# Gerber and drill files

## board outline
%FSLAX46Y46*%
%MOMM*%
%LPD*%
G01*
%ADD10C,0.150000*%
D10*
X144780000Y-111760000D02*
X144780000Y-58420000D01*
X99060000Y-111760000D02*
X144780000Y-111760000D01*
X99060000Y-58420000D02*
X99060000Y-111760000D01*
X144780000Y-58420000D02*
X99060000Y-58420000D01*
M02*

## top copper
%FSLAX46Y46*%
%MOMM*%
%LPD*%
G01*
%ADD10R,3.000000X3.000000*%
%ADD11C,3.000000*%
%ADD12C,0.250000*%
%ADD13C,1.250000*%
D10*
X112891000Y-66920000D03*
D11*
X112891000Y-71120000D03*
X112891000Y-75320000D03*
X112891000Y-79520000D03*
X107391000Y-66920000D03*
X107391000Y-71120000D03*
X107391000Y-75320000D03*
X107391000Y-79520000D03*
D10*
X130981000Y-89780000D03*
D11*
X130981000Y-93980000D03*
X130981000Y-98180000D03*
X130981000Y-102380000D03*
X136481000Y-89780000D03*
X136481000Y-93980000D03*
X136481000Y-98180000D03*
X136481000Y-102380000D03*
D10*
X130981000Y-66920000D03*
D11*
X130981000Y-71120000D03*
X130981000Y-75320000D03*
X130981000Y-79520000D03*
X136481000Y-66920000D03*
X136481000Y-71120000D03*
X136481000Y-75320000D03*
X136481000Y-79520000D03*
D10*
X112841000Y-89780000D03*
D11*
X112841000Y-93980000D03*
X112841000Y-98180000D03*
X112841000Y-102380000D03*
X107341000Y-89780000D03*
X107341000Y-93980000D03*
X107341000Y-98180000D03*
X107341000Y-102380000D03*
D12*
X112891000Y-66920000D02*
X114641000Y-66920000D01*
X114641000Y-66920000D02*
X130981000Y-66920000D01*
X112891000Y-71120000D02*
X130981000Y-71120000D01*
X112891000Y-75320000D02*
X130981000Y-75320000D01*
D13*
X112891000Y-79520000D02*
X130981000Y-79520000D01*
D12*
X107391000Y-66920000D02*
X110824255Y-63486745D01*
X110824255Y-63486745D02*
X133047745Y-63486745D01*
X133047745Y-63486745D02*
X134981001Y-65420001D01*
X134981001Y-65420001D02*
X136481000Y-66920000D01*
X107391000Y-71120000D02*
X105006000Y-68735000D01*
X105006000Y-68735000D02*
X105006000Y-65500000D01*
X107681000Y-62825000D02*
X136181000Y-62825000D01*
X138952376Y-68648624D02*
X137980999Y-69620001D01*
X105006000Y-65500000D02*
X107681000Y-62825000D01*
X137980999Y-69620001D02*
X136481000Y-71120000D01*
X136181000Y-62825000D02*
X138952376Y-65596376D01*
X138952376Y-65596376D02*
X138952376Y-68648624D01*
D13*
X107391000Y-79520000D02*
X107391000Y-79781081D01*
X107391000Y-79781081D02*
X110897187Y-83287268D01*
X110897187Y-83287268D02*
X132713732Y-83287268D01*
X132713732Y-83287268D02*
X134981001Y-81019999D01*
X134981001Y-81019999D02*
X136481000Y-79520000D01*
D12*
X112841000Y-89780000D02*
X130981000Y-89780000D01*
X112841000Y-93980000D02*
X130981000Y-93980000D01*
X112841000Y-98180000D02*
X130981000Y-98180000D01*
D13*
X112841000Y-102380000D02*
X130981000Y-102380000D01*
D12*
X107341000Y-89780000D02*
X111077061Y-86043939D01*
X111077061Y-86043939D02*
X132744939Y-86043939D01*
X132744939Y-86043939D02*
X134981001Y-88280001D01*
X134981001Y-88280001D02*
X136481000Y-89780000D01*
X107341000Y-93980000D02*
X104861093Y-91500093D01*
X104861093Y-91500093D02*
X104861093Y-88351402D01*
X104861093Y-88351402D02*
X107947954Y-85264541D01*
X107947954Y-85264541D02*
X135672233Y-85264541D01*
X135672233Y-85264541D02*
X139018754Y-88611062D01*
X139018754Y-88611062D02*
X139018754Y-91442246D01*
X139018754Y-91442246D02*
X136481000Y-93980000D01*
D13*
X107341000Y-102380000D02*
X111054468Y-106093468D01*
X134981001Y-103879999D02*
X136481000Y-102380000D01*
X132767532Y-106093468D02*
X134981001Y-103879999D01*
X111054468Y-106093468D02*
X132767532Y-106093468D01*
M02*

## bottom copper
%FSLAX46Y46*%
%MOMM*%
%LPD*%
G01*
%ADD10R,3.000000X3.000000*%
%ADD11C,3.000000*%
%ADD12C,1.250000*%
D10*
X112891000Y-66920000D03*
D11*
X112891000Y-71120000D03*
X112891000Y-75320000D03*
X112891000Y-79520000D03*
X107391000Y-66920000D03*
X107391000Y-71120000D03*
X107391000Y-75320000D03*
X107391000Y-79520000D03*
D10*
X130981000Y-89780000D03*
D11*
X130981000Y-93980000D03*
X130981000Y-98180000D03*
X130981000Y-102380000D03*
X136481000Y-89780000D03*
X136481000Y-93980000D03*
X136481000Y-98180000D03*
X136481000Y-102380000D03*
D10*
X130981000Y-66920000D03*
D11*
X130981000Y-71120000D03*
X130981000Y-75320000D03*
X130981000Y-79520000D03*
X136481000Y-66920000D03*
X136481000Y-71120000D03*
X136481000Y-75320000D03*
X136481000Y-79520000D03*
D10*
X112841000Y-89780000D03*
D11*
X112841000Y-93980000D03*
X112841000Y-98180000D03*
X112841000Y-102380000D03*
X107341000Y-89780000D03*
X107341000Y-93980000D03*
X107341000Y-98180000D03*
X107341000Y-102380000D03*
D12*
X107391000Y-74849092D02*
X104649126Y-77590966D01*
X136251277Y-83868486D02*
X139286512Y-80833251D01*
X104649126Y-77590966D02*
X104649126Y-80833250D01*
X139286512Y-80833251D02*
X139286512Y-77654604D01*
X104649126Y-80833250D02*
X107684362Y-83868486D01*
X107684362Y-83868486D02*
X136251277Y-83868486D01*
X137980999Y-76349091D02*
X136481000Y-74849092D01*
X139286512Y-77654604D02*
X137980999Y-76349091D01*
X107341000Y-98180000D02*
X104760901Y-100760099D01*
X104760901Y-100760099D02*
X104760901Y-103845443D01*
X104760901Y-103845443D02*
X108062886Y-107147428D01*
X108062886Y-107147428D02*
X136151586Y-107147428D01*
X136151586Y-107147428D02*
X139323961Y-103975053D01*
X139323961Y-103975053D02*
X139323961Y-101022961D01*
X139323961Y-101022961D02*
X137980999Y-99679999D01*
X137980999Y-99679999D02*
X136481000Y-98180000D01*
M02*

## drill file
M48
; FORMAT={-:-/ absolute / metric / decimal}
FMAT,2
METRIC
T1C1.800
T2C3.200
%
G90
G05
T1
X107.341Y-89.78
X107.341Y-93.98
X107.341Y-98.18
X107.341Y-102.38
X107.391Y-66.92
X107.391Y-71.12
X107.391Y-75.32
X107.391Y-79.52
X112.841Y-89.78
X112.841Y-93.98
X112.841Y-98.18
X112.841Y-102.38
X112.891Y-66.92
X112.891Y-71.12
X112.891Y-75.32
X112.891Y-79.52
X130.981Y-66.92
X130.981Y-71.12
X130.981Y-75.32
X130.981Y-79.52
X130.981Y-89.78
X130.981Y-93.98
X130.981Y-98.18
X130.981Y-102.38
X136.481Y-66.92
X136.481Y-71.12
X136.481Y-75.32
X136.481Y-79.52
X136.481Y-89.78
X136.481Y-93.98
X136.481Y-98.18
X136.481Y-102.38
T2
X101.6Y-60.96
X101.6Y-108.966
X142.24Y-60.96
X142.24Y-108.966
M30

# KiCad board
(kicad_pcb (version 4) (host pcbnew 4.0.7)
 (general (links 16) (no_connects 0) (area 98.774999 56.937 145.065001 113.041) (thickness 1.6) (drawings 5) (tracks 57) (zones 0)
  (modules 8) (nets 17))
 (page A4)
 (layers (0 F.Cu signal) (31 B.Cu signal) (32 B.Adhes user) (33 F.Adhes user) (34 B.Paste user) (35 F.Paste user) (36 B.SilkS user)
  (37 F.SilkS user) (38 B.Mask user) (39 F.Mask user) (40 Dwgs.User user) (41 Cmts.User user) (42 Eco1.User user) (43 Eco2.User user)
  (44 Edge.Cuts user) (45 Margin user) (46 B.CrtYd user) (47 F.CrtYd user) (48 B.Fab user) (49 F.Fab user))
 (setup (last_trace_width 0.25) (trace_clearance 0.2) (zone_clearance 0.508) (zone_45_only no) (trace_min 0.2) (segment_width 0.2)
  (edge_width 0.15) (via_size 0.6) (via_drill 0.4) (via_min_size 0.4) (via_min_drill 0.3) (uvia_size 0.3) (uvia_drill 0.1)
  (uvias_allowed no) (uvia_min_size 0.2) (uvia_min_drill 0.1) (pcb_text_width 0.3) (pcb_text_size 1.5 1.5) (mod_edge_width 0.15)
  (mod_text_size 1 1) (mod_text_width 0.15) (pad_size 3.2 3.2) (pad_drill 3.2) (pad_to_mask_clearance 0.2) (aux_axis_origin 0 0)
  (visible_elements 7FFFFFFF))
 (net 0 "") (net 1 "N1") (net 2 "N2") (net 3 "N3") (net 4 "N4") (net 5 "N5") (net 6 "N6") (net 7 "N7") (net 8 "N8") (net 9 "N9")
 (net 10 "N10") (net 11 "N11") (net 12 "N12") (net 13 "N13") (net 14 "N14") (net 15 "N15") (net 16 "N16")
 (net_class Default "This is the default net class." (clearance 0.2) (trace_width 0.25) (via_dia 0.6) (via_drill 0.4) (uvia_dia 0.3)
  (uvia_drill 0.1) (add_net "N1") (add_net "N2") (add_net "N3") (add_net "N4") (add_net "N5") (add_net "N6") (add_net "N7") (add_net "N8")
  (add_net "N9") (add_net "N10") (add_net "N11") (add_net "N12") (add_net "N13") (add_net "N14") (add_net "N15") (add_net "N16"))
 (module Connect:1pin (layer F.Cu) (at 142.24 108.966)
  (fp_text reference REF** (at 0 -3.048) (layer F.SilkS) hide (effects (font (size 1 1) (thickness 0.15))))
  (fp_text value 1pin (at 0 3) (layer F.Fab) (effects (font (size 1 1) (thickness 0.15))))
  (pad "" np_thru_hole circle (at 0 0) (size 3.2 3.2) (drill 3.2) (layers *.Cu *.Mask)))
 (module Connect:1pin (layer F.Cu) (at 101.6 108.966)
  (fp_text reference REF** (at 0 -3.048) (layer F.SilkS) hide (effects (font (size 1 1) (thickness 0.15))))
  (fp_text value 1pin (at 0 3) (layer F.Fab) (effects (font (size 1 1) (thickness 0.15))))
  (pad "" np_thru_hole circle (at 0 0) (size 3.2 3.2) (drill 3.2) (layers *.Cu *.Mask)))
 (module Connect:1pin (layer F.Cu) (at 101.6 60.96)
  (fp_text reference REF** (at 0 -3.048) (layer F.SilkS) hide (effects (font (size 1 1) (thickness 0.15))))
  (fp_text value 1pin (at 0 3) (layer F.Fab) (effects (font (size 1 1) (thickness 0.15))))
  (pad "" np_thru_hole circle (at 0 0) (size 3.2 3.2) (drill 3.2) (layers *.Cu *.Mask)))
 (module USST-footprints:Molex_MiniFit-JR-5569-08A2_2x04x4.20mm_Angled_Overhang (layer F.Cu) (at 112.891 66.92 270)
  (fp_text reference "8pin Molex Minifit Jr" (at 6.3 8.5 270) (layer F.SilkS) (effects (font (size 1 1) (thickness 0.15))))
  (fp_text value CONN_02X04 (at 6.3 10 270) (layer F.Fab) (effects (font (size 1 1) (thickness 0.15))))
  (pad 1 thru_hole rect (at 0 0 270) (size 3 3) (drill 1.8) (layers *.Cu *.Mask) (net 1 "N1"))
  (pad 2 thru_hole circle (at 4.2 0 270) (size 3 3) (drill 1.8) (layers *.Cu *.Mask) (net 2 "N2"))
  (pad 3 thru_hole circle (at 8.4 0 270) (size 3 3) (drill 1.8) (layers *.Cu *.Mask) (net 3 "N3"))
  (pad 4 thru_hole circle (at 12.6 0 270) (size 3 3) (drill 1.8) (layers *.Cu *.Mask) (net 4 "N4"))
  (pad 5 thru_hole circle (at 0 5.5 270) (size 3 3) (drill 1.8) (layers *.Cu *.Mask) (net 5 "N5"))
  (pad 6 thru_hole circle (at 4.2 5.5 270) (size 3 3) (drill 1.8) (layers *.Cu *.Mask) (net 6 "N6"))
  (pad 7 thru_hole circle (at 8.4 5.5 270) (size 3 3) (drill 1.8) (layers *.Cu *.Mask) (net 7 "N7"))
  (pad 8 thru_hole circle (at 12.6 5.5 270) (size 3 3) (drill 1.8) (layers *.Cu *.Mask) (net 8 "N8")))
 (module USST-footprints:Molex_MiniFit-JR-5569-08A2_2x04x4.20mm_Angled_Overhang (layer B.Cu) (at 130.981 89.78 270)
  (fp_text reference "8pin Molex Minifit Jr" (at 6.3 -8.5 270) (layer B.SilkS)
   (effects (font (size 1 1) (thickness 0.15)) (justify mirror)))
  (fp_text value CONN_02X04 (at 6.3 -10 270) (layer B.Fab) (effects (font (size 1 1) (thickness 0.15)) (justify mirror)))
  (pad 1 thru_hole rect (at 0 0 270) (size 3 3) (drill 1.8) (layers *.Cu *.Mask) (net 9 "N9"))
  (pad 2 thru_hole circle (at 4.2 0 270) (size 3 3) (drill 1.8) (layers *.Cu *.Mask) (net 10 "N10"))
  (pad 3 thru_hole circle (at 8.4 0 270) (size 3 3) (drill 1.8) (layers *.Cu *.Mask) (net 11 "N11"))
  (pad 4 thru_hole circle (at 12.6 0 270) (size 3 3) (drill 1.8) (layers *.Cu *.Mask) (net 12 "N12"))
  (pad 5 thru_hole circle (at 0 -5.5 270) (size 3 3) (drill 1.8) (layers *.Cu *.Mask) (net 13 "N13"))
  (pad 6 thru_hole circle (at 4.2 -5.5 270) (size 3 3) (drill 1.8) (layers *.Cu *.Mask) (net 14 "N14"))
  (pad 7 thru_hole circle (at 8.4 -5.5 270) (size 3 3) (drill 1.8) (layers *.Cu *.Mask) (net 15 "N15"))
  (pad 8 thru_hole circle (at 12.6 -5.5 270) (size 3 3) (drill 1.8) (layers *.Cu *.Mask) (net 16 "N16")))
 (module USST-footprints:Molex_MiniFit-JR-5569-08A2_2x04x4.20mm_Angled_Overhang (layer B.Cu) (at 130.981 66.92 270)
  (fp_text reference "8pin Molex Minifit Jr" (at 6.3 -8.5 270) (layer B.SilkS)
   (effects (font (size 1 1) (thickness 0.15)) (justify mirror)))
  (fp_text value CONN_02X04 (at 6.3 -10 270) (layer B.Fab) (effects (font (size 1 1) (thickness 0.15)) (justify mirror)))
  (pad 1 thru_hole rect (at 0 0 270) (size 3 3) (drill 1.8) (layers *.Cu *.Mask) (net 1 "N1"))
  (pad 2 thru_hole circle (at 4.2 0 270) (size 3 3) (drill 1.8) (layers *.Cu *.Mask) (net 2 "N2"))
  (pad 3 thru_hole circle (at 8.4 0 270) (size 3 3) (drill 1.8) (layers *.Cu *.Mask) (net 3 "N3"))
  (pad 4 thru_hole circle (at 12.6 0 270) (size 3 3) (drill 1.8) (layers *.Cu *.Mask) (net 4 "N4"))
  (pad 5 thru_hole circle (at 0 -5.5 270) (size 3 3) (drill 1.8) (layers *.Cu *.Mask) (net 5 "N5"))
  (pad 6 thru_hole circle (at 4.2 -5.5 270) (size 3 3) (drill 1.8) (layers *.Cu *.Mask) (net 6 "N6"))
  (pad 7 thru_hole circle (at 8.4 -5.5 270) (size 3 3) (drill 1.8) (layers *.Cu *.Mask) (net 7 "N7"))
  (pad 8 thru_hole circle (at 12.6 -5.5 270) (size 3 3) (drill 1.8) (layers *.Cu *.Mask) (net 8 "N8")))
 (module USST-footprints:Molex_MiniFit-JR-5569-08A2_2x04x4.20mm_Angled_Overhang (layer F.Cu) (at 112.841 89.78 270)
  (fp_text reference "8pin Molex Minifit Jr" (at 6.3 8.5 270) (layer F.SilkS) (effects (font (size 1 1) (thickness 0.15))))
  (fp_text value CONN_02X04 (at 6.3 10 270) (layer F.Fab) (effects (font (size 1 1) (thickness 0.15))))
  (pad 1 thru_hole rect (at 0 0 270) (size 3 3) (drill 1.8) (layers *.Cu *.Mask) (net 9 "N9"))
  (pad 2 thru_hole circle (at 4.2 0 270) (size 3 3) (drill 1.8) (layers *.Cu *.Mask) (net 10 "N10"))
  (pad 3 thru_hole circle (at 8.4 0 270) (size 3 3) (drill 1.8) (layers *.Cu *.Mask) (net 11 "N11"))
  (pad 4 thru_hole circle (at 12.6 0 270) (size 3 3) (drill 1.8) (layers *.Cu *.Mask) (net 12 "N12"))
  (pad 5 thru_hole circle (at 0 5.5 270) (size 3 3) (drill 1.8) (layers *.Cu *.Mask) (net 13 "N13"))
  (pad 6 thru_hole circle (at 4.2 5.5 270) (size 3 3) (drill 1.8) (layers *.Cu *.Mask) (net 14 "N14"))
  (pad 7 thru_hole circle (at 8.4 5.5 270) (size 3 3) (drill 1.8) (layers *.Cu *.Mask) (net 15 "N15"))
  (pad 8 thru_hole circle (at 12.6 5.5 270) (size 3 3) (drill 1.8) (layers *.Cu *.Mask) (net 16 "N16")))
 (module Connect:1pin (layer F.Cu) (at 142.24 60.96)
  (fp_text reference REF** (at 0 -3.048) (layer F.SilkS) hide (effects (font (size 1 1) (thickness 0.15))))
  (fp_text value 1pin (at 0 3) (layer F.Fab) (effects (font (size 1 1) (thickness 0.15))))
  (pad "" np_thru_hole circle (at 0 0) (size 3.2 3.2) (drill 3.2) (layers *.Cu *.Mask)))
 (gr_line (start 144.78 111.76) (end 144.78 58.42) (layer Edge.Cuts) (width 0.15))
 (gr_line (start 99.06 111.76) (end 144.78 111.76) (layer Edge.Cuts) (width 0.15))
 (gr_line (start 99.06 58.42) (end 99.06 111.76) (layer Edge.Cuts) (width 0.15))
 (gr_line (start 144.78 58.42) (end 99.06 58.42) (layer Edge.Cuts) (width 0.15))
 (segment (start 112.891 66.92) (end 114.641 66.92) (width 0.25) (layer F.Cu) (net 1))
 (segment (start 114.641 66.92) (end 130.981 66.92) (width 0.25) (layer F.Cu) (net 1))
 (segment (start 112.891 71.12) (end 130.981 71.12) (width 0.25) (layer F.Cu) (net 2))
 (segment (start 112.891 75.32) (end 130.981 75.32) (width 0.25) (layer F.Cu) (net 3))
 (segment (start 112.891 79.52) (end 130.981 79.52) (width 1.25) (layer F.Cu) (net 4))
 (segment (start 107.391 66.92) (end 110.824255 63.486745) (width 0.25) (layer F.Cu) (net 5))
 (segment (start 110.824255 63.486745) (end 133.047745 63.486745) (width 0.25) (layer F.Cu) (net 5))
 (segment (start 133.047745 63.486745) (end 134.981001 65.420001) (width 0.25) (layer F.Cu) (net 5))
 (segment (start 134.981001 65.420001) (end 136.481 66.92) (width 0.25) (layer F.Cu) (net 5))
 (segment (start 107.391 71.12) (end 105.006 68.735) (width 0.25) (layer F.Cu) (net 6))
 (segment (start 105.006 68.735) (end 105.006 65.5) (width 0.25) (layer F.Cu) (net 6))
 (segment (start 107.681 62.825) (end 136.181 62.825) (width 0.25) (layer F.Cu) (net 6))
 (segment (start 138.952376 68.648624) (end 137.980999 69.620001) (width 0.25) (layer F.Cu) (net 6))
 (segment (start 105.006 65.5) (end 107.681 62.825) (width 0.25) (layer F.Cu) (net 6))
 (segment (start 137.980999 69.620001) (end 136.481 71.12) (width 0.25) (layer F.Cu) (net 6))
 (segment (start 136.181 62.825) (end 138.952376 65.596376) (width 0.25) (layer F.Cu) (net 6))
 (segment (start 138.952376 65.596376) (end 138.952376 68.648624) (width 0.25) (layer F.Cu) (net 6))
 (segment (start 107.391 74.849092) (end 104.649126 77.590966) (width 1.25) (layer B.Cu) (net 7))
 (segment (start 136.251277 83.868486) (end 139.286512 80.833251) (width 1.25) (layer B.Cu) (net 7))
 (segment (start 104.649126 77.590966) (end 104.649126 80.83325) (width 1.25) (layer B.Cu) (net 7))
 (segment (start 139.286512 80.833251) (end 139.286512 77.654604) (width 1.25) (layer B.Cu) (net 7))
 (segment (start 104.649126 80.83325) (end 107.684362 83.868486) (width 1.25) (layer B.Cu) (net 7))
 (segment (start 107.684362 83.868486) (end 136.251277 83.868486) (width 1.25) (layer B.Cu) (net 7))
 (segment (start 137.980999 76.349091) (end 136.481 74.849092) (width 1.25) (layer B.Cu) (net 7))
 (segment (start 139.286512 77.654604) (end 137.980999 76.349091) (width 1.25) (layer B.Cu) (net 7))
 (segment (start 107.391 79.52) (end 107.391 79.781081) (width 1.25) (layer F.Cu) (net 8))
 (segment (start 107.391 79.781081) (end 110.897187 83.287268) (width 1.25) (layer F.Cu) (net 8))
 (segment (start 110.897187 83.287268) (end 132.713732 83.287268) (width 1.25) (layer F.Cu) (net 8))
 (segment (start 132.713732 83.287268) (end 134.981001 81.019999) (width 1.25) (layer F.Cu) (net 8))
 (segment (start 134.981001 81.019999) (end 136.481 79.52) (width 1.25) (layer F.Cu) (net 8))
 (segment (start 112.841 89.78) (end 130.981 89.78) (width 0.25) (layer F.Cu) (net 9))
 (segment (start 112.841 93.98) (end 130.981 93.98) (width 0.25) (layer F.Cu) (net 10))
 (segment (start 112.841 98.18) (end 130.981 98.18) (width 0.25) (layer F.Cu) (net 11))
 (segment (start 112.841 102.38) (end 130.981 102.38) (width 1.25) (layer F.Cu) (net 12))
 (segment (start 107.341 89.78) (end 111.077061 86.043939) (width 0.25) (layer F.Cu) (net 13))
 (segment (start 111.077061 86.043939) (end 132.744939 86.043939) (width 0.25) (layer F.Cu) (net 13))
 (segment (start 132.744939 86.043939) (end 134.981001 88.280001) (width 0.25) (layer F.Cu) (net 13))
 (segment (start 134.981001 88.280001) (end 136.481 89.78) (width 0.25) (layer F.Cu) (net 13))
 (segment (start 107.341 93.98) (end 104.861093 91.500093) (width 0.25) (layer F.Cu) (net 14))
 (segment (start 104.861093 91.500093) (end 104.861093 88.351402) (width 0.25) (layer F.Cu) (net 14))
 (segment (start 104.861093 88.351402) (end 107.947954 85.264541) (width 0.25) (layer F.Cu) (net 14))
 (segment (start 107.947954 85.264541) (end 135.672233 85.264541) (width 0.25) (layer F.Cu) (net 14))
 (segment (start 135.672233 85.264541) (end 139.018754 88.611062) (width 0.25) (layer F.Cu) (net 14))
 (segment (start 139.018754 88.611062) (end 139.018754 91.442246) (width 0.25) (layer F.Cu) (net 14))
 (segment (start 139.018754 91.442246) (end 136.481 93.98) (width 0.25) (layer F.Cu) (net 14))
 (segment (start 107.341 98.18) (end 104.760901 100.760099) (width 1.25) (layer B.Cu) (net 15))
 (segment (start 104.760901 100.760099) (end 104.760901 103.845443) (width 1.25) (layer B.Cu) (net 15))
 (segment (start 104.760901 103.845443) (end 108.062886 107.147428) (width 1.25) (layer B.Cu) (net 15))
 (segment (start 108.062886 107.147428) (end 136.151586 107.147428) (width 1.25) (layer B.Cu) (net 15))
 (segment (start 136.151586 107.147428) (end 139.323961 103.975053) (width 1.25) (layer B.Cu) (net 15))
 (segment (start 139.323961 103.975053) (end 139.323961 101.022961) (width 1.25) (layer B.Cu) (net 15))
 (segment (start 139.323961 101.022961) (end 137.980999 99.679999) (width 1.25) (layer B.Cu) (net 15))
 (segment (start 137.980999 99.679999) (end 136.481 98.18) (width 1.25) (layer B.Cu) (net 15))
 (segment (start 107.341 102.38) (end 111.054468 106.093468) (width 1.25) (layer F.Cu) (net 16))
 (segment (start 134.981001 103.879999) (end 136.481 102.38) (width 1.25) (layer F.Cu) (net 16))
 (segment (start 132.767532 106.093468) (end 134.981001 103.879999) (width 1.25) (layer F.Cu) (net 16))
 (segment (start 111.054468 106.093468) (end 132.767532 106.093468) (width 1.25) (layer F.Cu) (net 16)))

